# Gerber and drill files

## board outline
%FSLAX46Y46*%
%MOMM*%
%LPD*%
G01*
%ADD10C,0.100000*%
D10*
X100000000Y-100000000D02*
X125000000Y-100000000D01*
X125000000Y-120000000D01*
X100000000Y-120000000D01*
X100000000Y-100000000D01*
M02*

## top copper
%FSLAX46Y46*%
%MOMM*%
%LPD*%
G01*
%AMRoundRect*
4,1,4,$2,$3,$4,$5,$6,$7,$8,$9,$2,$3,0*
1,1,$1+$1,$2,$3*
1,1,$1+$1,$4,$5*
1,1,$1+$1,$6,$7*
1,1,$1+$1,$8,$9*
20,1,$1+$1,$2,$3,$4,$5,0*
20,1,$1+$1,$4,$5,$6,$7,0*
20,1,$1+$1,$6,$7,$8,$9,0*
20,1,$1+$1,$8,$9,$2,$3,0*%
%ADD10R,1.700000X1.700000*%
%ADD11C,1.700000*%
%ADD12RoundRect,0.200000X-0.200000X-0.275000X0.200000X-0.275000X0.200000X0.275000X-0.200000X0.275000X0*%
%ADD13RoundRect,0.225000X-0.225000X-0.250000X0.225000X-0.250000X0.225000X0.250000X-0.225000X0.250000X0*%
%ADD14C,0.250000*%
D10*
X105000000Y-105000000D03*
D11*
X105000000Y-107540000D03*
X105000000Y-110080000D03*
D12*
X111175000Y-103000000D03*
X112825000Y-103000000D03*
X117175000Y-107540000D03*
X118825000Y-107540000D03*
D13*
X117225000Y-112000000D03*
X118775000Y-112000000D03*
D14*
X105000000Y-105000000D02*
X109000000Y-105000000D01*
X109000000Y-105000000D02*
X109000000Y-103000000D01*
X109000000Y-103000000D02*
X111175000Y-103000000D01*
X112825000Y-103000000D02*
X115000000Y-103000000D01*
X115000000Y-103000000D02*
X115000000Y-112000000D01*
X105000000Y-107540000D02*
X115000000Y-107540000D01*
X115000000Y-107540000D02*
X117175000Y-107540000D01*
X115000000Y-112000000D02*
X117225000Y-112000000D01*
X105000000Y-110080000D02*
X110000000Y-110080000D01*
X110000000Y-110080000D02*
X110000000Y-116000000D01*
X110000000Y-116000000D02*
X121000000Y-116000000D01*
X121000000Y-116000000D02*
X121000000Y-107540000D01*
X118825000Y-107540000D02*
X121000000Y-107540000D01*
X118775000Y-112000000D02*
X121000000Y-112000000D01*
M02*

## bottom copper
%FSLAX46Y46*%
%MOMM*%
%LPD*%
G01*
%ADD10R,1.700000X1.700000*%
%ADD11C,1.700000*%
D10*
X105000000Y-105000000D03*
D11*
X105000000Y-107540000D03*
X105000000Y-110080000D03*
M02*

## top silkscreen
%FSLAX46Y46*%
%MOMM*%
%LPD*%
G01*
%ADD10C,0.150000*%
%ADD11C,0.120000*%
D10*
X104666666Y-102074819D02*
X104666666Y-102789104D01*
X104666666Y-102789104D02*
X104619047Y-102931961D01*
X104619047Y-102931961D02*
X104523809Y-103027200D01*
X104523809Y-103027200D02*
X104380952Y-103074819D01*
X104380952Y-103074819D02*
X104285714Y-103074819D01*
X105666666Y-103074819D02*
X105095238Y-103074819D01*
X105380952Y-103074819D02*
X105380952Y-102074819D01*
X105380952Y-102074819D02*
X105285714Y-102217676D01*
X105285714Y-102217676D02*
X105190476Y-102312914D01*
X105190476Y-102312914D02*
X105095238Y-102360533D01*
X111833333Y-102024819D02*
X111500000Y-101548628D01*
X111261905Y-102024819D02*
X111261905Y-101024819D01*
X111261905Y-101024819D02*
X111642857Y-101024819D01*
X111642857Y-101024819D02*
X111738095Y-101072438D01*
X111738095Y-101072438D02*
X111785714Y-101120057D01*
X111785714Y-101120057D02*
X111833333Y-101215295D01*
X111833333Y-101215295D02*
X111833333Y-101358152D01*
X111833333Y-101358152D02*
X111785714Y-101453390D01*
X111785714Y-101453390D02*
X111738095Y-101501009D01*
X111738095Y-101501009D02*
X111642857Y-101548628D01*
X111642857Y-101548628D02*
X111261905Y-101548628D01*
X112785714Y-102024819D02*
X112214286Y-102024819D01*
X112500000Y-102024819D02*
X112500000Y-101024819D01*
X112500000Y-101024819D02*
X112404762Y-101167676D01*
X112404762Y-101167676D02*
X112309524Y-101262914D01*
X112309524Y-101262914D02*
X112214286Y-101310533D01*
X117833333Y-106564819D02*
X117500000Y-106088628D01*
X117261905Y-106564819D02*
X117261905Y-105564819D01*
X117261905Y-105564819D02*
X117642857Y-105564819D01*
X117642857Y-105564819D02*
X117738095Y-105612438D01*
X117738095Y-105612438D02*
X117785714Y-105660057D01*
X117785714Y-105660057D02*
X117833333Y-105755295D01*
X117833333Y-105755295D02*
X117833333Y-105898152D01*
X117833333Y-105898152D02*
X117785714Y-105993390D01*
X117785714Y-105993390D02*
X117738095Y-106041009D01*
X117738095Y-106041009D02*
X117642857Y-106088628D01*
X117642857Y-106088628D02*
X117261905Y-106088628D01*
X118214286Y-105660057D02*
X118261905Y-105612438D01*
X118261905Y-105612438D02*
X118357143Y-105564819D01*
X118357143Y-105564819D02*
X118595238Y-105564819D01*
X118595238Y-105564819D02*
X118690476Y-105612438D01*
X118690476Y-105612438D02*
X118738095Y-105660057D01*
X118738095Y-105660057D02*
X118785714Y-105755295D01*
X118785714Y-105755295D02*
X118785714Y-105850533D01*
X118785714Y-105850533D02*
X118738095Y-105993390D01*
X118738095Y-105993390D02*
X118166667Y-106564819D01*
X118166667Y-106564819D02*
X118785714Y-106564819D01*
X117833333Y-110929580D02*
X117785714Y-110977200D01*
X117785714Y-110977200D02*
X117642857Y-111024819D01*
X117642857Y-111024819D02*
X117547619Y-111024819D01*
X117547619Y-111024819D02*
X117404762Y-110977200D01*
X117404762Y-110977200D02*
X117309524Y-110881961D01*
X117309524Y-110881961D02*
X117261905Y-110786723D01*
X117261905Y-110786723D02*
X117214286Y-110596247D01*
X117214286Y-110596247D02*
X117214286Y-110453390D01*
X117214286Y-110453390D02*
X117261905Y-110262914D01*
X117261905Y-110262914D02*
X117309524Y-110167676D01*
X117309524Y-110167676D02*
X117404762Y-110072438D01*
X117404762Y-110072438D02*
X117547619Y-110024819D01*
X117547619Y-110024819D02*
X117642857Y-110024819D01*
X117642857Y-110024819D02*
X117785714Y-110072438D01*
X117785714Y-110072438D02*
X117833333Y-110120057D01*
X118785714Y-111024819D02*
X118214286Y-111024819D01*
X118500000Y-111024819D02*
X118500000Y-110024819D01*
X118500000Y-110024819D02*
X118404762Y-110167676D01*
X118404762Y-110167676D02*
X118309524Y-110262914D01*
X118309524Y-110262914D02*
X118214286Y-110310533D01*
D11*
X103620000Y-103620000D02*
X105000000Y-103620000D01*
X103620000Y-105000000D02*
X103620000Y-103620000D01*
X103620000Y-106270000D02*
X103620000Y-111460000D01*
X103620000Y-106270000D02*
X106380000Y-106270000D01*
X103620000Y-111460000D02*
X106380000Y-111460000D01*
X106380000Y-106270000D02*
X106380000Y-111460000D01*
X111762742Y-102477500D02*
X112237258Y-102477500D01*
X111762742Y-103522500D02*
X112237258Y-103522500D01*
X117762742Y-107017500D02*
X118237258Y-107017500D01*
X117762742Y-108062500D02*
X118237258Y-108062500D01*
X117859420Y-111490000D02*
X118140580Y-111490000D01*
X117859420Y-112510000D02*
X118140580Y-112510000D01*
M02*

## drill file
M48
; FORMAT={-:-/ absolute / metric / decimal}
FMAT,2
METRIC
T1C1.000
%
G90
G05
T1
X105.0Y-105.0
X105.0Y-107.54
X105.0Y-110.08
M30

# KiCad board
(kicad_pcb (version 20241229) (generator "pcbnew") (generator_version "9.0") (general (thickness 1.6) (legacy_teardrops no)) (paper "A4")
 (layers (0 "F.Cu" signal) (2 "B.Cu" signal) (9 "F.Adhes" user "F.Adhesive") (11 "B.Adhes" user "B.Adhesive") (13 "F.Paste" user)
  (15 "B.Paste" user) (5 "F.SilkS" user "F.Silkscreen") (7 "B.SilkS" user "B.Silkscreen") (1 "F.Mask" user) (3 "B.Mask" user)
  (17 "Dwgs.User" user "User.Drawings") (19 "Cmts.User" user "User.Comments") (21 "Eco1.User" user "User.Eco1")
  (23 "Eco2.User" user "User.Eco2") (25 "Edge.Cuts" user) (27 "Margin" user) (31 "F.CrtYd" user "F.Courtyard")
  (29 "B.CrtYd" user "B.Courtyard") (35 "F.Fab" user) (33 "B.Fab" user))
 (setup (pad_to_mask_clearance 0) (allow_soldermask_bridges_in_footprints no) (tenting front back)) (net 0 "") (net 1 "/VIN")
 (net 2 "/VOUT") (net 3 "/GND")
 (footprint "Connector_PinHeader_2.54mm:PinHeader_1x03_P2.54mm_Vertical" (layer "F.Cu") (at 105 105)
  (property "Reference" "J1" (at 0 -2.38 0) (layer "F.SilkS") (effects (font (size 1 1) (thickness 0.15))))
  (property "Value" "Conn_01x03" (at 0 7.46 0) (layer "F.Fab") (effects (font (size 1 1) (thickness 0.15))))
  (fp_line (start -1.38 -1.38) (end 0 -1.38) (stroke (width 0.12) (type solid)) (layer "F.SilkS"))
  (fp_line (start -1.38 0) (end -1.38 -1.38) (stroke (width 0.12) (type solid)) (layer "F.SilkS"))
  (fp_line (start -1.38 1.27) (end -1.38 6.46) (stroke (width 0.12) (type solid)) (layer "F.SilkS"))
  (fp_line (start -1.38 1.27) (end 1.38 1.27) (stroke (width 0.12) (type solid)) (layer "F.SilkS"))
  (fp_line (start -1.38 6.46) (end 1.38 6.46) (stroke (width 0.12) (type solid)) (layer "F.SilkS"))
  (fp_line (start 1.38 1.27) (end 1.38 6.46) (stroke (width 0.12) (type solid)) (layer "F.SilkS"))
  (pad "1" thru_hole rect (at 0 0) (size 1.7 1.7) (drill 1) (layers "*.Cu" "*.Mask") (remove_unused_layers no) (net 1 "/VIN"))
  (pad "2" thru_hole circle (at 0 2.54) (size 1.7 1.7) (drill 1) (layers "*.Cu" "*.Mask") (remove_unused_layers no) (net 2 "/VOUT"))
  (pad "3" thru_hole circle (at 0 5.08) (size 1.7 1.7) (drill 1) (layers "*.Cu" "*.Mask") (remove_unused_layers no) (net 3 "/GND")))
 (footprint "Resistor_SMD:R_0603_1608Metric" (layer "F.Cu") (at 112 103)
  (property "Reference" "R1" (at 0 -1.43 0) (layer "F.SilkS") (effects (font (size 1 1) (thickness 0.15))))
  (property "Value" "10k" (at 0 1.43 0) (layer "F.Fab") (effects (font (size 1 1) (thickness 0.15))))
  (fp_line (start -0.237258 -0.5225) (end 0.237258 -0.5225) (stroke (width 0.12) (type solid)) (layer "F.SilkS"))
  (fp_line (start -0.237258 0.5225) (end 0.237258 0.5225) (stroke (width 0.12) (type solid)) (layer "F.SilkS"))
  (pad "1" smd roundrect (at -0.825 0) (size 0.8 0.95) (layers "F.Cu" "F.Mask" "F.Paste") (roundrect_rratio 0.25) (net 1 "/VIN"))
  (pad "2" smd roundrect (at 0.825 0) (size 0.8 0.95) (layers "F.Cu" "F.Mask" "F.Paste") (roundrect_rratio 0.25) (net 2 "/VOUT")))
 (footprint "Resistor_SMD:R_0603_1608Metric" (layer "F.Cu") (at 118 107.54)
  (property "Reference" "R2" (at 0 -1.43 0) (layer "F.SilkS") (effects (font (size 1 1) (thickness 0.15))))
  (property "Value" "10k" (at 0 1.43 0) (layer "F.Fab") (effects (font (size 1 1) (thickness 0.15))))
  (fp_line (start -0.237258 -0.5225) (end 0.237258 -0.5225) (stroke (width 0.12) (type solid)) (layer "F.SilkS"))
  (fp_line (start -0.237258 0.5225) (end 0.237258 0.5225) (stroke (width 0.12) (type solid)) (layer "F.SilkS"))
  (pad "1" smd roundrect (at -0.825 0) (size 0.8 0.95) (layers "F.Cu" "F.Mask" "F.Paste") (roundrect_rratio 0.25) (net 2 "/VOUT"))
  (pad "2" smd roundrect (at 0.825 0) (size 0.8 0.95) (layers "F.Cu" "F.Mask" "F.Paste") (roundrect_rratio 0.25) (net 3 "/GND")))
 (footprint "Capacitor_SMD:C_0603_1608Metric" (layer "F.Cu") (at 118 112)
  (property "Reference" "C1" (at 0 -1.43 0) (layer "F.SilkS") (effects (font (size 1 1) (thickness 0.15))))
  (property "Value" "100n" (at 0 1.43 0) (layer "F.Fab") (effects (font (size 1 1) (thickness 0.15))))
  (fp_line (start -0.14058 -0.51) (end 0.14058 -0.51) (stroke (width 0.12) (type solid)) (layer "F.SilkS"))
  (fp_line (start -0.14058 0.51) (end 0.14058 0.51) (stroke (width 0.12) (type solid)) (layer "F.SilkS"))
  (pad "1" smd roundrect (at -0.775 0) (size 0.9 0.95) (layers "F.Cu" "F.Mask" "F.Paste") (roundrect_rratio 0.25) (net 2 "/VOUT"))
  (pad "2" smd roundrect (at 0.775 0) (size 0.9 0.95) (layers "F.Cu" "F.Mask" "F.Paste") (roundrect_rratio 0.25) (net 3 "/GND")))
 (gr_rect (start 100 100) (end 125 120) (stroke (width 0.1) (type default)) (fill no) (layer "Edge.Cuts"))
 (segment (start 105 105) (end 109 105) (width 0.25) (layer "F.Cu") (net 1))
 (segment (start 109 105) (end 109 103) (width 0.25) (layer "F.Cu") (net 1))
 (segment (start 109 103) (end 111.175 103) (width 0.25) (layer "F.Cu") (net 1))
 (segment (start 112.825 103) (end 115 103) (width 0.25) (layer "F.Cu") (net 2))
 (segment (start 115 103) (end 115 112) (width 0.25) (layer "F.Cu") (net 2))
 (segment (start 105 107.54) (end 115 107.54) (width 0.25) (layer "F.Cu") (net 2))
 (segment (start 115 107.54) (end 117.175 107.54) (width 0.25) (layer "F.Cu") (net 2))
 (segment (start 115 112) (end 117.225 112) (width 0.25) (layer "F.Cu") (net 2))
 (segment (start 105 110.08) (end 110 110.08) (width 0.25) (layer "F.Cu") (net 3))
 (segment (start 110 110.08) (end 110 116) (width 0.25) (layer "F.Cu") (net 3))
 (segment (start 110 116) (end 121 116) (width 0.25) (layer "F.Cu") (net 3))
 (segment (start 121 116) (end 121 107.54) (width 0.25) (layer "F.Cu") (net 3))
 (segment (start 118.825 107.54) (end 121 107.54) (width 0.25) (layer "F.Cu") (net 3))
 (segment (start 118.775 112) (end 121 112) (width 0.25) (layer "F.Cu") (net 3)))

